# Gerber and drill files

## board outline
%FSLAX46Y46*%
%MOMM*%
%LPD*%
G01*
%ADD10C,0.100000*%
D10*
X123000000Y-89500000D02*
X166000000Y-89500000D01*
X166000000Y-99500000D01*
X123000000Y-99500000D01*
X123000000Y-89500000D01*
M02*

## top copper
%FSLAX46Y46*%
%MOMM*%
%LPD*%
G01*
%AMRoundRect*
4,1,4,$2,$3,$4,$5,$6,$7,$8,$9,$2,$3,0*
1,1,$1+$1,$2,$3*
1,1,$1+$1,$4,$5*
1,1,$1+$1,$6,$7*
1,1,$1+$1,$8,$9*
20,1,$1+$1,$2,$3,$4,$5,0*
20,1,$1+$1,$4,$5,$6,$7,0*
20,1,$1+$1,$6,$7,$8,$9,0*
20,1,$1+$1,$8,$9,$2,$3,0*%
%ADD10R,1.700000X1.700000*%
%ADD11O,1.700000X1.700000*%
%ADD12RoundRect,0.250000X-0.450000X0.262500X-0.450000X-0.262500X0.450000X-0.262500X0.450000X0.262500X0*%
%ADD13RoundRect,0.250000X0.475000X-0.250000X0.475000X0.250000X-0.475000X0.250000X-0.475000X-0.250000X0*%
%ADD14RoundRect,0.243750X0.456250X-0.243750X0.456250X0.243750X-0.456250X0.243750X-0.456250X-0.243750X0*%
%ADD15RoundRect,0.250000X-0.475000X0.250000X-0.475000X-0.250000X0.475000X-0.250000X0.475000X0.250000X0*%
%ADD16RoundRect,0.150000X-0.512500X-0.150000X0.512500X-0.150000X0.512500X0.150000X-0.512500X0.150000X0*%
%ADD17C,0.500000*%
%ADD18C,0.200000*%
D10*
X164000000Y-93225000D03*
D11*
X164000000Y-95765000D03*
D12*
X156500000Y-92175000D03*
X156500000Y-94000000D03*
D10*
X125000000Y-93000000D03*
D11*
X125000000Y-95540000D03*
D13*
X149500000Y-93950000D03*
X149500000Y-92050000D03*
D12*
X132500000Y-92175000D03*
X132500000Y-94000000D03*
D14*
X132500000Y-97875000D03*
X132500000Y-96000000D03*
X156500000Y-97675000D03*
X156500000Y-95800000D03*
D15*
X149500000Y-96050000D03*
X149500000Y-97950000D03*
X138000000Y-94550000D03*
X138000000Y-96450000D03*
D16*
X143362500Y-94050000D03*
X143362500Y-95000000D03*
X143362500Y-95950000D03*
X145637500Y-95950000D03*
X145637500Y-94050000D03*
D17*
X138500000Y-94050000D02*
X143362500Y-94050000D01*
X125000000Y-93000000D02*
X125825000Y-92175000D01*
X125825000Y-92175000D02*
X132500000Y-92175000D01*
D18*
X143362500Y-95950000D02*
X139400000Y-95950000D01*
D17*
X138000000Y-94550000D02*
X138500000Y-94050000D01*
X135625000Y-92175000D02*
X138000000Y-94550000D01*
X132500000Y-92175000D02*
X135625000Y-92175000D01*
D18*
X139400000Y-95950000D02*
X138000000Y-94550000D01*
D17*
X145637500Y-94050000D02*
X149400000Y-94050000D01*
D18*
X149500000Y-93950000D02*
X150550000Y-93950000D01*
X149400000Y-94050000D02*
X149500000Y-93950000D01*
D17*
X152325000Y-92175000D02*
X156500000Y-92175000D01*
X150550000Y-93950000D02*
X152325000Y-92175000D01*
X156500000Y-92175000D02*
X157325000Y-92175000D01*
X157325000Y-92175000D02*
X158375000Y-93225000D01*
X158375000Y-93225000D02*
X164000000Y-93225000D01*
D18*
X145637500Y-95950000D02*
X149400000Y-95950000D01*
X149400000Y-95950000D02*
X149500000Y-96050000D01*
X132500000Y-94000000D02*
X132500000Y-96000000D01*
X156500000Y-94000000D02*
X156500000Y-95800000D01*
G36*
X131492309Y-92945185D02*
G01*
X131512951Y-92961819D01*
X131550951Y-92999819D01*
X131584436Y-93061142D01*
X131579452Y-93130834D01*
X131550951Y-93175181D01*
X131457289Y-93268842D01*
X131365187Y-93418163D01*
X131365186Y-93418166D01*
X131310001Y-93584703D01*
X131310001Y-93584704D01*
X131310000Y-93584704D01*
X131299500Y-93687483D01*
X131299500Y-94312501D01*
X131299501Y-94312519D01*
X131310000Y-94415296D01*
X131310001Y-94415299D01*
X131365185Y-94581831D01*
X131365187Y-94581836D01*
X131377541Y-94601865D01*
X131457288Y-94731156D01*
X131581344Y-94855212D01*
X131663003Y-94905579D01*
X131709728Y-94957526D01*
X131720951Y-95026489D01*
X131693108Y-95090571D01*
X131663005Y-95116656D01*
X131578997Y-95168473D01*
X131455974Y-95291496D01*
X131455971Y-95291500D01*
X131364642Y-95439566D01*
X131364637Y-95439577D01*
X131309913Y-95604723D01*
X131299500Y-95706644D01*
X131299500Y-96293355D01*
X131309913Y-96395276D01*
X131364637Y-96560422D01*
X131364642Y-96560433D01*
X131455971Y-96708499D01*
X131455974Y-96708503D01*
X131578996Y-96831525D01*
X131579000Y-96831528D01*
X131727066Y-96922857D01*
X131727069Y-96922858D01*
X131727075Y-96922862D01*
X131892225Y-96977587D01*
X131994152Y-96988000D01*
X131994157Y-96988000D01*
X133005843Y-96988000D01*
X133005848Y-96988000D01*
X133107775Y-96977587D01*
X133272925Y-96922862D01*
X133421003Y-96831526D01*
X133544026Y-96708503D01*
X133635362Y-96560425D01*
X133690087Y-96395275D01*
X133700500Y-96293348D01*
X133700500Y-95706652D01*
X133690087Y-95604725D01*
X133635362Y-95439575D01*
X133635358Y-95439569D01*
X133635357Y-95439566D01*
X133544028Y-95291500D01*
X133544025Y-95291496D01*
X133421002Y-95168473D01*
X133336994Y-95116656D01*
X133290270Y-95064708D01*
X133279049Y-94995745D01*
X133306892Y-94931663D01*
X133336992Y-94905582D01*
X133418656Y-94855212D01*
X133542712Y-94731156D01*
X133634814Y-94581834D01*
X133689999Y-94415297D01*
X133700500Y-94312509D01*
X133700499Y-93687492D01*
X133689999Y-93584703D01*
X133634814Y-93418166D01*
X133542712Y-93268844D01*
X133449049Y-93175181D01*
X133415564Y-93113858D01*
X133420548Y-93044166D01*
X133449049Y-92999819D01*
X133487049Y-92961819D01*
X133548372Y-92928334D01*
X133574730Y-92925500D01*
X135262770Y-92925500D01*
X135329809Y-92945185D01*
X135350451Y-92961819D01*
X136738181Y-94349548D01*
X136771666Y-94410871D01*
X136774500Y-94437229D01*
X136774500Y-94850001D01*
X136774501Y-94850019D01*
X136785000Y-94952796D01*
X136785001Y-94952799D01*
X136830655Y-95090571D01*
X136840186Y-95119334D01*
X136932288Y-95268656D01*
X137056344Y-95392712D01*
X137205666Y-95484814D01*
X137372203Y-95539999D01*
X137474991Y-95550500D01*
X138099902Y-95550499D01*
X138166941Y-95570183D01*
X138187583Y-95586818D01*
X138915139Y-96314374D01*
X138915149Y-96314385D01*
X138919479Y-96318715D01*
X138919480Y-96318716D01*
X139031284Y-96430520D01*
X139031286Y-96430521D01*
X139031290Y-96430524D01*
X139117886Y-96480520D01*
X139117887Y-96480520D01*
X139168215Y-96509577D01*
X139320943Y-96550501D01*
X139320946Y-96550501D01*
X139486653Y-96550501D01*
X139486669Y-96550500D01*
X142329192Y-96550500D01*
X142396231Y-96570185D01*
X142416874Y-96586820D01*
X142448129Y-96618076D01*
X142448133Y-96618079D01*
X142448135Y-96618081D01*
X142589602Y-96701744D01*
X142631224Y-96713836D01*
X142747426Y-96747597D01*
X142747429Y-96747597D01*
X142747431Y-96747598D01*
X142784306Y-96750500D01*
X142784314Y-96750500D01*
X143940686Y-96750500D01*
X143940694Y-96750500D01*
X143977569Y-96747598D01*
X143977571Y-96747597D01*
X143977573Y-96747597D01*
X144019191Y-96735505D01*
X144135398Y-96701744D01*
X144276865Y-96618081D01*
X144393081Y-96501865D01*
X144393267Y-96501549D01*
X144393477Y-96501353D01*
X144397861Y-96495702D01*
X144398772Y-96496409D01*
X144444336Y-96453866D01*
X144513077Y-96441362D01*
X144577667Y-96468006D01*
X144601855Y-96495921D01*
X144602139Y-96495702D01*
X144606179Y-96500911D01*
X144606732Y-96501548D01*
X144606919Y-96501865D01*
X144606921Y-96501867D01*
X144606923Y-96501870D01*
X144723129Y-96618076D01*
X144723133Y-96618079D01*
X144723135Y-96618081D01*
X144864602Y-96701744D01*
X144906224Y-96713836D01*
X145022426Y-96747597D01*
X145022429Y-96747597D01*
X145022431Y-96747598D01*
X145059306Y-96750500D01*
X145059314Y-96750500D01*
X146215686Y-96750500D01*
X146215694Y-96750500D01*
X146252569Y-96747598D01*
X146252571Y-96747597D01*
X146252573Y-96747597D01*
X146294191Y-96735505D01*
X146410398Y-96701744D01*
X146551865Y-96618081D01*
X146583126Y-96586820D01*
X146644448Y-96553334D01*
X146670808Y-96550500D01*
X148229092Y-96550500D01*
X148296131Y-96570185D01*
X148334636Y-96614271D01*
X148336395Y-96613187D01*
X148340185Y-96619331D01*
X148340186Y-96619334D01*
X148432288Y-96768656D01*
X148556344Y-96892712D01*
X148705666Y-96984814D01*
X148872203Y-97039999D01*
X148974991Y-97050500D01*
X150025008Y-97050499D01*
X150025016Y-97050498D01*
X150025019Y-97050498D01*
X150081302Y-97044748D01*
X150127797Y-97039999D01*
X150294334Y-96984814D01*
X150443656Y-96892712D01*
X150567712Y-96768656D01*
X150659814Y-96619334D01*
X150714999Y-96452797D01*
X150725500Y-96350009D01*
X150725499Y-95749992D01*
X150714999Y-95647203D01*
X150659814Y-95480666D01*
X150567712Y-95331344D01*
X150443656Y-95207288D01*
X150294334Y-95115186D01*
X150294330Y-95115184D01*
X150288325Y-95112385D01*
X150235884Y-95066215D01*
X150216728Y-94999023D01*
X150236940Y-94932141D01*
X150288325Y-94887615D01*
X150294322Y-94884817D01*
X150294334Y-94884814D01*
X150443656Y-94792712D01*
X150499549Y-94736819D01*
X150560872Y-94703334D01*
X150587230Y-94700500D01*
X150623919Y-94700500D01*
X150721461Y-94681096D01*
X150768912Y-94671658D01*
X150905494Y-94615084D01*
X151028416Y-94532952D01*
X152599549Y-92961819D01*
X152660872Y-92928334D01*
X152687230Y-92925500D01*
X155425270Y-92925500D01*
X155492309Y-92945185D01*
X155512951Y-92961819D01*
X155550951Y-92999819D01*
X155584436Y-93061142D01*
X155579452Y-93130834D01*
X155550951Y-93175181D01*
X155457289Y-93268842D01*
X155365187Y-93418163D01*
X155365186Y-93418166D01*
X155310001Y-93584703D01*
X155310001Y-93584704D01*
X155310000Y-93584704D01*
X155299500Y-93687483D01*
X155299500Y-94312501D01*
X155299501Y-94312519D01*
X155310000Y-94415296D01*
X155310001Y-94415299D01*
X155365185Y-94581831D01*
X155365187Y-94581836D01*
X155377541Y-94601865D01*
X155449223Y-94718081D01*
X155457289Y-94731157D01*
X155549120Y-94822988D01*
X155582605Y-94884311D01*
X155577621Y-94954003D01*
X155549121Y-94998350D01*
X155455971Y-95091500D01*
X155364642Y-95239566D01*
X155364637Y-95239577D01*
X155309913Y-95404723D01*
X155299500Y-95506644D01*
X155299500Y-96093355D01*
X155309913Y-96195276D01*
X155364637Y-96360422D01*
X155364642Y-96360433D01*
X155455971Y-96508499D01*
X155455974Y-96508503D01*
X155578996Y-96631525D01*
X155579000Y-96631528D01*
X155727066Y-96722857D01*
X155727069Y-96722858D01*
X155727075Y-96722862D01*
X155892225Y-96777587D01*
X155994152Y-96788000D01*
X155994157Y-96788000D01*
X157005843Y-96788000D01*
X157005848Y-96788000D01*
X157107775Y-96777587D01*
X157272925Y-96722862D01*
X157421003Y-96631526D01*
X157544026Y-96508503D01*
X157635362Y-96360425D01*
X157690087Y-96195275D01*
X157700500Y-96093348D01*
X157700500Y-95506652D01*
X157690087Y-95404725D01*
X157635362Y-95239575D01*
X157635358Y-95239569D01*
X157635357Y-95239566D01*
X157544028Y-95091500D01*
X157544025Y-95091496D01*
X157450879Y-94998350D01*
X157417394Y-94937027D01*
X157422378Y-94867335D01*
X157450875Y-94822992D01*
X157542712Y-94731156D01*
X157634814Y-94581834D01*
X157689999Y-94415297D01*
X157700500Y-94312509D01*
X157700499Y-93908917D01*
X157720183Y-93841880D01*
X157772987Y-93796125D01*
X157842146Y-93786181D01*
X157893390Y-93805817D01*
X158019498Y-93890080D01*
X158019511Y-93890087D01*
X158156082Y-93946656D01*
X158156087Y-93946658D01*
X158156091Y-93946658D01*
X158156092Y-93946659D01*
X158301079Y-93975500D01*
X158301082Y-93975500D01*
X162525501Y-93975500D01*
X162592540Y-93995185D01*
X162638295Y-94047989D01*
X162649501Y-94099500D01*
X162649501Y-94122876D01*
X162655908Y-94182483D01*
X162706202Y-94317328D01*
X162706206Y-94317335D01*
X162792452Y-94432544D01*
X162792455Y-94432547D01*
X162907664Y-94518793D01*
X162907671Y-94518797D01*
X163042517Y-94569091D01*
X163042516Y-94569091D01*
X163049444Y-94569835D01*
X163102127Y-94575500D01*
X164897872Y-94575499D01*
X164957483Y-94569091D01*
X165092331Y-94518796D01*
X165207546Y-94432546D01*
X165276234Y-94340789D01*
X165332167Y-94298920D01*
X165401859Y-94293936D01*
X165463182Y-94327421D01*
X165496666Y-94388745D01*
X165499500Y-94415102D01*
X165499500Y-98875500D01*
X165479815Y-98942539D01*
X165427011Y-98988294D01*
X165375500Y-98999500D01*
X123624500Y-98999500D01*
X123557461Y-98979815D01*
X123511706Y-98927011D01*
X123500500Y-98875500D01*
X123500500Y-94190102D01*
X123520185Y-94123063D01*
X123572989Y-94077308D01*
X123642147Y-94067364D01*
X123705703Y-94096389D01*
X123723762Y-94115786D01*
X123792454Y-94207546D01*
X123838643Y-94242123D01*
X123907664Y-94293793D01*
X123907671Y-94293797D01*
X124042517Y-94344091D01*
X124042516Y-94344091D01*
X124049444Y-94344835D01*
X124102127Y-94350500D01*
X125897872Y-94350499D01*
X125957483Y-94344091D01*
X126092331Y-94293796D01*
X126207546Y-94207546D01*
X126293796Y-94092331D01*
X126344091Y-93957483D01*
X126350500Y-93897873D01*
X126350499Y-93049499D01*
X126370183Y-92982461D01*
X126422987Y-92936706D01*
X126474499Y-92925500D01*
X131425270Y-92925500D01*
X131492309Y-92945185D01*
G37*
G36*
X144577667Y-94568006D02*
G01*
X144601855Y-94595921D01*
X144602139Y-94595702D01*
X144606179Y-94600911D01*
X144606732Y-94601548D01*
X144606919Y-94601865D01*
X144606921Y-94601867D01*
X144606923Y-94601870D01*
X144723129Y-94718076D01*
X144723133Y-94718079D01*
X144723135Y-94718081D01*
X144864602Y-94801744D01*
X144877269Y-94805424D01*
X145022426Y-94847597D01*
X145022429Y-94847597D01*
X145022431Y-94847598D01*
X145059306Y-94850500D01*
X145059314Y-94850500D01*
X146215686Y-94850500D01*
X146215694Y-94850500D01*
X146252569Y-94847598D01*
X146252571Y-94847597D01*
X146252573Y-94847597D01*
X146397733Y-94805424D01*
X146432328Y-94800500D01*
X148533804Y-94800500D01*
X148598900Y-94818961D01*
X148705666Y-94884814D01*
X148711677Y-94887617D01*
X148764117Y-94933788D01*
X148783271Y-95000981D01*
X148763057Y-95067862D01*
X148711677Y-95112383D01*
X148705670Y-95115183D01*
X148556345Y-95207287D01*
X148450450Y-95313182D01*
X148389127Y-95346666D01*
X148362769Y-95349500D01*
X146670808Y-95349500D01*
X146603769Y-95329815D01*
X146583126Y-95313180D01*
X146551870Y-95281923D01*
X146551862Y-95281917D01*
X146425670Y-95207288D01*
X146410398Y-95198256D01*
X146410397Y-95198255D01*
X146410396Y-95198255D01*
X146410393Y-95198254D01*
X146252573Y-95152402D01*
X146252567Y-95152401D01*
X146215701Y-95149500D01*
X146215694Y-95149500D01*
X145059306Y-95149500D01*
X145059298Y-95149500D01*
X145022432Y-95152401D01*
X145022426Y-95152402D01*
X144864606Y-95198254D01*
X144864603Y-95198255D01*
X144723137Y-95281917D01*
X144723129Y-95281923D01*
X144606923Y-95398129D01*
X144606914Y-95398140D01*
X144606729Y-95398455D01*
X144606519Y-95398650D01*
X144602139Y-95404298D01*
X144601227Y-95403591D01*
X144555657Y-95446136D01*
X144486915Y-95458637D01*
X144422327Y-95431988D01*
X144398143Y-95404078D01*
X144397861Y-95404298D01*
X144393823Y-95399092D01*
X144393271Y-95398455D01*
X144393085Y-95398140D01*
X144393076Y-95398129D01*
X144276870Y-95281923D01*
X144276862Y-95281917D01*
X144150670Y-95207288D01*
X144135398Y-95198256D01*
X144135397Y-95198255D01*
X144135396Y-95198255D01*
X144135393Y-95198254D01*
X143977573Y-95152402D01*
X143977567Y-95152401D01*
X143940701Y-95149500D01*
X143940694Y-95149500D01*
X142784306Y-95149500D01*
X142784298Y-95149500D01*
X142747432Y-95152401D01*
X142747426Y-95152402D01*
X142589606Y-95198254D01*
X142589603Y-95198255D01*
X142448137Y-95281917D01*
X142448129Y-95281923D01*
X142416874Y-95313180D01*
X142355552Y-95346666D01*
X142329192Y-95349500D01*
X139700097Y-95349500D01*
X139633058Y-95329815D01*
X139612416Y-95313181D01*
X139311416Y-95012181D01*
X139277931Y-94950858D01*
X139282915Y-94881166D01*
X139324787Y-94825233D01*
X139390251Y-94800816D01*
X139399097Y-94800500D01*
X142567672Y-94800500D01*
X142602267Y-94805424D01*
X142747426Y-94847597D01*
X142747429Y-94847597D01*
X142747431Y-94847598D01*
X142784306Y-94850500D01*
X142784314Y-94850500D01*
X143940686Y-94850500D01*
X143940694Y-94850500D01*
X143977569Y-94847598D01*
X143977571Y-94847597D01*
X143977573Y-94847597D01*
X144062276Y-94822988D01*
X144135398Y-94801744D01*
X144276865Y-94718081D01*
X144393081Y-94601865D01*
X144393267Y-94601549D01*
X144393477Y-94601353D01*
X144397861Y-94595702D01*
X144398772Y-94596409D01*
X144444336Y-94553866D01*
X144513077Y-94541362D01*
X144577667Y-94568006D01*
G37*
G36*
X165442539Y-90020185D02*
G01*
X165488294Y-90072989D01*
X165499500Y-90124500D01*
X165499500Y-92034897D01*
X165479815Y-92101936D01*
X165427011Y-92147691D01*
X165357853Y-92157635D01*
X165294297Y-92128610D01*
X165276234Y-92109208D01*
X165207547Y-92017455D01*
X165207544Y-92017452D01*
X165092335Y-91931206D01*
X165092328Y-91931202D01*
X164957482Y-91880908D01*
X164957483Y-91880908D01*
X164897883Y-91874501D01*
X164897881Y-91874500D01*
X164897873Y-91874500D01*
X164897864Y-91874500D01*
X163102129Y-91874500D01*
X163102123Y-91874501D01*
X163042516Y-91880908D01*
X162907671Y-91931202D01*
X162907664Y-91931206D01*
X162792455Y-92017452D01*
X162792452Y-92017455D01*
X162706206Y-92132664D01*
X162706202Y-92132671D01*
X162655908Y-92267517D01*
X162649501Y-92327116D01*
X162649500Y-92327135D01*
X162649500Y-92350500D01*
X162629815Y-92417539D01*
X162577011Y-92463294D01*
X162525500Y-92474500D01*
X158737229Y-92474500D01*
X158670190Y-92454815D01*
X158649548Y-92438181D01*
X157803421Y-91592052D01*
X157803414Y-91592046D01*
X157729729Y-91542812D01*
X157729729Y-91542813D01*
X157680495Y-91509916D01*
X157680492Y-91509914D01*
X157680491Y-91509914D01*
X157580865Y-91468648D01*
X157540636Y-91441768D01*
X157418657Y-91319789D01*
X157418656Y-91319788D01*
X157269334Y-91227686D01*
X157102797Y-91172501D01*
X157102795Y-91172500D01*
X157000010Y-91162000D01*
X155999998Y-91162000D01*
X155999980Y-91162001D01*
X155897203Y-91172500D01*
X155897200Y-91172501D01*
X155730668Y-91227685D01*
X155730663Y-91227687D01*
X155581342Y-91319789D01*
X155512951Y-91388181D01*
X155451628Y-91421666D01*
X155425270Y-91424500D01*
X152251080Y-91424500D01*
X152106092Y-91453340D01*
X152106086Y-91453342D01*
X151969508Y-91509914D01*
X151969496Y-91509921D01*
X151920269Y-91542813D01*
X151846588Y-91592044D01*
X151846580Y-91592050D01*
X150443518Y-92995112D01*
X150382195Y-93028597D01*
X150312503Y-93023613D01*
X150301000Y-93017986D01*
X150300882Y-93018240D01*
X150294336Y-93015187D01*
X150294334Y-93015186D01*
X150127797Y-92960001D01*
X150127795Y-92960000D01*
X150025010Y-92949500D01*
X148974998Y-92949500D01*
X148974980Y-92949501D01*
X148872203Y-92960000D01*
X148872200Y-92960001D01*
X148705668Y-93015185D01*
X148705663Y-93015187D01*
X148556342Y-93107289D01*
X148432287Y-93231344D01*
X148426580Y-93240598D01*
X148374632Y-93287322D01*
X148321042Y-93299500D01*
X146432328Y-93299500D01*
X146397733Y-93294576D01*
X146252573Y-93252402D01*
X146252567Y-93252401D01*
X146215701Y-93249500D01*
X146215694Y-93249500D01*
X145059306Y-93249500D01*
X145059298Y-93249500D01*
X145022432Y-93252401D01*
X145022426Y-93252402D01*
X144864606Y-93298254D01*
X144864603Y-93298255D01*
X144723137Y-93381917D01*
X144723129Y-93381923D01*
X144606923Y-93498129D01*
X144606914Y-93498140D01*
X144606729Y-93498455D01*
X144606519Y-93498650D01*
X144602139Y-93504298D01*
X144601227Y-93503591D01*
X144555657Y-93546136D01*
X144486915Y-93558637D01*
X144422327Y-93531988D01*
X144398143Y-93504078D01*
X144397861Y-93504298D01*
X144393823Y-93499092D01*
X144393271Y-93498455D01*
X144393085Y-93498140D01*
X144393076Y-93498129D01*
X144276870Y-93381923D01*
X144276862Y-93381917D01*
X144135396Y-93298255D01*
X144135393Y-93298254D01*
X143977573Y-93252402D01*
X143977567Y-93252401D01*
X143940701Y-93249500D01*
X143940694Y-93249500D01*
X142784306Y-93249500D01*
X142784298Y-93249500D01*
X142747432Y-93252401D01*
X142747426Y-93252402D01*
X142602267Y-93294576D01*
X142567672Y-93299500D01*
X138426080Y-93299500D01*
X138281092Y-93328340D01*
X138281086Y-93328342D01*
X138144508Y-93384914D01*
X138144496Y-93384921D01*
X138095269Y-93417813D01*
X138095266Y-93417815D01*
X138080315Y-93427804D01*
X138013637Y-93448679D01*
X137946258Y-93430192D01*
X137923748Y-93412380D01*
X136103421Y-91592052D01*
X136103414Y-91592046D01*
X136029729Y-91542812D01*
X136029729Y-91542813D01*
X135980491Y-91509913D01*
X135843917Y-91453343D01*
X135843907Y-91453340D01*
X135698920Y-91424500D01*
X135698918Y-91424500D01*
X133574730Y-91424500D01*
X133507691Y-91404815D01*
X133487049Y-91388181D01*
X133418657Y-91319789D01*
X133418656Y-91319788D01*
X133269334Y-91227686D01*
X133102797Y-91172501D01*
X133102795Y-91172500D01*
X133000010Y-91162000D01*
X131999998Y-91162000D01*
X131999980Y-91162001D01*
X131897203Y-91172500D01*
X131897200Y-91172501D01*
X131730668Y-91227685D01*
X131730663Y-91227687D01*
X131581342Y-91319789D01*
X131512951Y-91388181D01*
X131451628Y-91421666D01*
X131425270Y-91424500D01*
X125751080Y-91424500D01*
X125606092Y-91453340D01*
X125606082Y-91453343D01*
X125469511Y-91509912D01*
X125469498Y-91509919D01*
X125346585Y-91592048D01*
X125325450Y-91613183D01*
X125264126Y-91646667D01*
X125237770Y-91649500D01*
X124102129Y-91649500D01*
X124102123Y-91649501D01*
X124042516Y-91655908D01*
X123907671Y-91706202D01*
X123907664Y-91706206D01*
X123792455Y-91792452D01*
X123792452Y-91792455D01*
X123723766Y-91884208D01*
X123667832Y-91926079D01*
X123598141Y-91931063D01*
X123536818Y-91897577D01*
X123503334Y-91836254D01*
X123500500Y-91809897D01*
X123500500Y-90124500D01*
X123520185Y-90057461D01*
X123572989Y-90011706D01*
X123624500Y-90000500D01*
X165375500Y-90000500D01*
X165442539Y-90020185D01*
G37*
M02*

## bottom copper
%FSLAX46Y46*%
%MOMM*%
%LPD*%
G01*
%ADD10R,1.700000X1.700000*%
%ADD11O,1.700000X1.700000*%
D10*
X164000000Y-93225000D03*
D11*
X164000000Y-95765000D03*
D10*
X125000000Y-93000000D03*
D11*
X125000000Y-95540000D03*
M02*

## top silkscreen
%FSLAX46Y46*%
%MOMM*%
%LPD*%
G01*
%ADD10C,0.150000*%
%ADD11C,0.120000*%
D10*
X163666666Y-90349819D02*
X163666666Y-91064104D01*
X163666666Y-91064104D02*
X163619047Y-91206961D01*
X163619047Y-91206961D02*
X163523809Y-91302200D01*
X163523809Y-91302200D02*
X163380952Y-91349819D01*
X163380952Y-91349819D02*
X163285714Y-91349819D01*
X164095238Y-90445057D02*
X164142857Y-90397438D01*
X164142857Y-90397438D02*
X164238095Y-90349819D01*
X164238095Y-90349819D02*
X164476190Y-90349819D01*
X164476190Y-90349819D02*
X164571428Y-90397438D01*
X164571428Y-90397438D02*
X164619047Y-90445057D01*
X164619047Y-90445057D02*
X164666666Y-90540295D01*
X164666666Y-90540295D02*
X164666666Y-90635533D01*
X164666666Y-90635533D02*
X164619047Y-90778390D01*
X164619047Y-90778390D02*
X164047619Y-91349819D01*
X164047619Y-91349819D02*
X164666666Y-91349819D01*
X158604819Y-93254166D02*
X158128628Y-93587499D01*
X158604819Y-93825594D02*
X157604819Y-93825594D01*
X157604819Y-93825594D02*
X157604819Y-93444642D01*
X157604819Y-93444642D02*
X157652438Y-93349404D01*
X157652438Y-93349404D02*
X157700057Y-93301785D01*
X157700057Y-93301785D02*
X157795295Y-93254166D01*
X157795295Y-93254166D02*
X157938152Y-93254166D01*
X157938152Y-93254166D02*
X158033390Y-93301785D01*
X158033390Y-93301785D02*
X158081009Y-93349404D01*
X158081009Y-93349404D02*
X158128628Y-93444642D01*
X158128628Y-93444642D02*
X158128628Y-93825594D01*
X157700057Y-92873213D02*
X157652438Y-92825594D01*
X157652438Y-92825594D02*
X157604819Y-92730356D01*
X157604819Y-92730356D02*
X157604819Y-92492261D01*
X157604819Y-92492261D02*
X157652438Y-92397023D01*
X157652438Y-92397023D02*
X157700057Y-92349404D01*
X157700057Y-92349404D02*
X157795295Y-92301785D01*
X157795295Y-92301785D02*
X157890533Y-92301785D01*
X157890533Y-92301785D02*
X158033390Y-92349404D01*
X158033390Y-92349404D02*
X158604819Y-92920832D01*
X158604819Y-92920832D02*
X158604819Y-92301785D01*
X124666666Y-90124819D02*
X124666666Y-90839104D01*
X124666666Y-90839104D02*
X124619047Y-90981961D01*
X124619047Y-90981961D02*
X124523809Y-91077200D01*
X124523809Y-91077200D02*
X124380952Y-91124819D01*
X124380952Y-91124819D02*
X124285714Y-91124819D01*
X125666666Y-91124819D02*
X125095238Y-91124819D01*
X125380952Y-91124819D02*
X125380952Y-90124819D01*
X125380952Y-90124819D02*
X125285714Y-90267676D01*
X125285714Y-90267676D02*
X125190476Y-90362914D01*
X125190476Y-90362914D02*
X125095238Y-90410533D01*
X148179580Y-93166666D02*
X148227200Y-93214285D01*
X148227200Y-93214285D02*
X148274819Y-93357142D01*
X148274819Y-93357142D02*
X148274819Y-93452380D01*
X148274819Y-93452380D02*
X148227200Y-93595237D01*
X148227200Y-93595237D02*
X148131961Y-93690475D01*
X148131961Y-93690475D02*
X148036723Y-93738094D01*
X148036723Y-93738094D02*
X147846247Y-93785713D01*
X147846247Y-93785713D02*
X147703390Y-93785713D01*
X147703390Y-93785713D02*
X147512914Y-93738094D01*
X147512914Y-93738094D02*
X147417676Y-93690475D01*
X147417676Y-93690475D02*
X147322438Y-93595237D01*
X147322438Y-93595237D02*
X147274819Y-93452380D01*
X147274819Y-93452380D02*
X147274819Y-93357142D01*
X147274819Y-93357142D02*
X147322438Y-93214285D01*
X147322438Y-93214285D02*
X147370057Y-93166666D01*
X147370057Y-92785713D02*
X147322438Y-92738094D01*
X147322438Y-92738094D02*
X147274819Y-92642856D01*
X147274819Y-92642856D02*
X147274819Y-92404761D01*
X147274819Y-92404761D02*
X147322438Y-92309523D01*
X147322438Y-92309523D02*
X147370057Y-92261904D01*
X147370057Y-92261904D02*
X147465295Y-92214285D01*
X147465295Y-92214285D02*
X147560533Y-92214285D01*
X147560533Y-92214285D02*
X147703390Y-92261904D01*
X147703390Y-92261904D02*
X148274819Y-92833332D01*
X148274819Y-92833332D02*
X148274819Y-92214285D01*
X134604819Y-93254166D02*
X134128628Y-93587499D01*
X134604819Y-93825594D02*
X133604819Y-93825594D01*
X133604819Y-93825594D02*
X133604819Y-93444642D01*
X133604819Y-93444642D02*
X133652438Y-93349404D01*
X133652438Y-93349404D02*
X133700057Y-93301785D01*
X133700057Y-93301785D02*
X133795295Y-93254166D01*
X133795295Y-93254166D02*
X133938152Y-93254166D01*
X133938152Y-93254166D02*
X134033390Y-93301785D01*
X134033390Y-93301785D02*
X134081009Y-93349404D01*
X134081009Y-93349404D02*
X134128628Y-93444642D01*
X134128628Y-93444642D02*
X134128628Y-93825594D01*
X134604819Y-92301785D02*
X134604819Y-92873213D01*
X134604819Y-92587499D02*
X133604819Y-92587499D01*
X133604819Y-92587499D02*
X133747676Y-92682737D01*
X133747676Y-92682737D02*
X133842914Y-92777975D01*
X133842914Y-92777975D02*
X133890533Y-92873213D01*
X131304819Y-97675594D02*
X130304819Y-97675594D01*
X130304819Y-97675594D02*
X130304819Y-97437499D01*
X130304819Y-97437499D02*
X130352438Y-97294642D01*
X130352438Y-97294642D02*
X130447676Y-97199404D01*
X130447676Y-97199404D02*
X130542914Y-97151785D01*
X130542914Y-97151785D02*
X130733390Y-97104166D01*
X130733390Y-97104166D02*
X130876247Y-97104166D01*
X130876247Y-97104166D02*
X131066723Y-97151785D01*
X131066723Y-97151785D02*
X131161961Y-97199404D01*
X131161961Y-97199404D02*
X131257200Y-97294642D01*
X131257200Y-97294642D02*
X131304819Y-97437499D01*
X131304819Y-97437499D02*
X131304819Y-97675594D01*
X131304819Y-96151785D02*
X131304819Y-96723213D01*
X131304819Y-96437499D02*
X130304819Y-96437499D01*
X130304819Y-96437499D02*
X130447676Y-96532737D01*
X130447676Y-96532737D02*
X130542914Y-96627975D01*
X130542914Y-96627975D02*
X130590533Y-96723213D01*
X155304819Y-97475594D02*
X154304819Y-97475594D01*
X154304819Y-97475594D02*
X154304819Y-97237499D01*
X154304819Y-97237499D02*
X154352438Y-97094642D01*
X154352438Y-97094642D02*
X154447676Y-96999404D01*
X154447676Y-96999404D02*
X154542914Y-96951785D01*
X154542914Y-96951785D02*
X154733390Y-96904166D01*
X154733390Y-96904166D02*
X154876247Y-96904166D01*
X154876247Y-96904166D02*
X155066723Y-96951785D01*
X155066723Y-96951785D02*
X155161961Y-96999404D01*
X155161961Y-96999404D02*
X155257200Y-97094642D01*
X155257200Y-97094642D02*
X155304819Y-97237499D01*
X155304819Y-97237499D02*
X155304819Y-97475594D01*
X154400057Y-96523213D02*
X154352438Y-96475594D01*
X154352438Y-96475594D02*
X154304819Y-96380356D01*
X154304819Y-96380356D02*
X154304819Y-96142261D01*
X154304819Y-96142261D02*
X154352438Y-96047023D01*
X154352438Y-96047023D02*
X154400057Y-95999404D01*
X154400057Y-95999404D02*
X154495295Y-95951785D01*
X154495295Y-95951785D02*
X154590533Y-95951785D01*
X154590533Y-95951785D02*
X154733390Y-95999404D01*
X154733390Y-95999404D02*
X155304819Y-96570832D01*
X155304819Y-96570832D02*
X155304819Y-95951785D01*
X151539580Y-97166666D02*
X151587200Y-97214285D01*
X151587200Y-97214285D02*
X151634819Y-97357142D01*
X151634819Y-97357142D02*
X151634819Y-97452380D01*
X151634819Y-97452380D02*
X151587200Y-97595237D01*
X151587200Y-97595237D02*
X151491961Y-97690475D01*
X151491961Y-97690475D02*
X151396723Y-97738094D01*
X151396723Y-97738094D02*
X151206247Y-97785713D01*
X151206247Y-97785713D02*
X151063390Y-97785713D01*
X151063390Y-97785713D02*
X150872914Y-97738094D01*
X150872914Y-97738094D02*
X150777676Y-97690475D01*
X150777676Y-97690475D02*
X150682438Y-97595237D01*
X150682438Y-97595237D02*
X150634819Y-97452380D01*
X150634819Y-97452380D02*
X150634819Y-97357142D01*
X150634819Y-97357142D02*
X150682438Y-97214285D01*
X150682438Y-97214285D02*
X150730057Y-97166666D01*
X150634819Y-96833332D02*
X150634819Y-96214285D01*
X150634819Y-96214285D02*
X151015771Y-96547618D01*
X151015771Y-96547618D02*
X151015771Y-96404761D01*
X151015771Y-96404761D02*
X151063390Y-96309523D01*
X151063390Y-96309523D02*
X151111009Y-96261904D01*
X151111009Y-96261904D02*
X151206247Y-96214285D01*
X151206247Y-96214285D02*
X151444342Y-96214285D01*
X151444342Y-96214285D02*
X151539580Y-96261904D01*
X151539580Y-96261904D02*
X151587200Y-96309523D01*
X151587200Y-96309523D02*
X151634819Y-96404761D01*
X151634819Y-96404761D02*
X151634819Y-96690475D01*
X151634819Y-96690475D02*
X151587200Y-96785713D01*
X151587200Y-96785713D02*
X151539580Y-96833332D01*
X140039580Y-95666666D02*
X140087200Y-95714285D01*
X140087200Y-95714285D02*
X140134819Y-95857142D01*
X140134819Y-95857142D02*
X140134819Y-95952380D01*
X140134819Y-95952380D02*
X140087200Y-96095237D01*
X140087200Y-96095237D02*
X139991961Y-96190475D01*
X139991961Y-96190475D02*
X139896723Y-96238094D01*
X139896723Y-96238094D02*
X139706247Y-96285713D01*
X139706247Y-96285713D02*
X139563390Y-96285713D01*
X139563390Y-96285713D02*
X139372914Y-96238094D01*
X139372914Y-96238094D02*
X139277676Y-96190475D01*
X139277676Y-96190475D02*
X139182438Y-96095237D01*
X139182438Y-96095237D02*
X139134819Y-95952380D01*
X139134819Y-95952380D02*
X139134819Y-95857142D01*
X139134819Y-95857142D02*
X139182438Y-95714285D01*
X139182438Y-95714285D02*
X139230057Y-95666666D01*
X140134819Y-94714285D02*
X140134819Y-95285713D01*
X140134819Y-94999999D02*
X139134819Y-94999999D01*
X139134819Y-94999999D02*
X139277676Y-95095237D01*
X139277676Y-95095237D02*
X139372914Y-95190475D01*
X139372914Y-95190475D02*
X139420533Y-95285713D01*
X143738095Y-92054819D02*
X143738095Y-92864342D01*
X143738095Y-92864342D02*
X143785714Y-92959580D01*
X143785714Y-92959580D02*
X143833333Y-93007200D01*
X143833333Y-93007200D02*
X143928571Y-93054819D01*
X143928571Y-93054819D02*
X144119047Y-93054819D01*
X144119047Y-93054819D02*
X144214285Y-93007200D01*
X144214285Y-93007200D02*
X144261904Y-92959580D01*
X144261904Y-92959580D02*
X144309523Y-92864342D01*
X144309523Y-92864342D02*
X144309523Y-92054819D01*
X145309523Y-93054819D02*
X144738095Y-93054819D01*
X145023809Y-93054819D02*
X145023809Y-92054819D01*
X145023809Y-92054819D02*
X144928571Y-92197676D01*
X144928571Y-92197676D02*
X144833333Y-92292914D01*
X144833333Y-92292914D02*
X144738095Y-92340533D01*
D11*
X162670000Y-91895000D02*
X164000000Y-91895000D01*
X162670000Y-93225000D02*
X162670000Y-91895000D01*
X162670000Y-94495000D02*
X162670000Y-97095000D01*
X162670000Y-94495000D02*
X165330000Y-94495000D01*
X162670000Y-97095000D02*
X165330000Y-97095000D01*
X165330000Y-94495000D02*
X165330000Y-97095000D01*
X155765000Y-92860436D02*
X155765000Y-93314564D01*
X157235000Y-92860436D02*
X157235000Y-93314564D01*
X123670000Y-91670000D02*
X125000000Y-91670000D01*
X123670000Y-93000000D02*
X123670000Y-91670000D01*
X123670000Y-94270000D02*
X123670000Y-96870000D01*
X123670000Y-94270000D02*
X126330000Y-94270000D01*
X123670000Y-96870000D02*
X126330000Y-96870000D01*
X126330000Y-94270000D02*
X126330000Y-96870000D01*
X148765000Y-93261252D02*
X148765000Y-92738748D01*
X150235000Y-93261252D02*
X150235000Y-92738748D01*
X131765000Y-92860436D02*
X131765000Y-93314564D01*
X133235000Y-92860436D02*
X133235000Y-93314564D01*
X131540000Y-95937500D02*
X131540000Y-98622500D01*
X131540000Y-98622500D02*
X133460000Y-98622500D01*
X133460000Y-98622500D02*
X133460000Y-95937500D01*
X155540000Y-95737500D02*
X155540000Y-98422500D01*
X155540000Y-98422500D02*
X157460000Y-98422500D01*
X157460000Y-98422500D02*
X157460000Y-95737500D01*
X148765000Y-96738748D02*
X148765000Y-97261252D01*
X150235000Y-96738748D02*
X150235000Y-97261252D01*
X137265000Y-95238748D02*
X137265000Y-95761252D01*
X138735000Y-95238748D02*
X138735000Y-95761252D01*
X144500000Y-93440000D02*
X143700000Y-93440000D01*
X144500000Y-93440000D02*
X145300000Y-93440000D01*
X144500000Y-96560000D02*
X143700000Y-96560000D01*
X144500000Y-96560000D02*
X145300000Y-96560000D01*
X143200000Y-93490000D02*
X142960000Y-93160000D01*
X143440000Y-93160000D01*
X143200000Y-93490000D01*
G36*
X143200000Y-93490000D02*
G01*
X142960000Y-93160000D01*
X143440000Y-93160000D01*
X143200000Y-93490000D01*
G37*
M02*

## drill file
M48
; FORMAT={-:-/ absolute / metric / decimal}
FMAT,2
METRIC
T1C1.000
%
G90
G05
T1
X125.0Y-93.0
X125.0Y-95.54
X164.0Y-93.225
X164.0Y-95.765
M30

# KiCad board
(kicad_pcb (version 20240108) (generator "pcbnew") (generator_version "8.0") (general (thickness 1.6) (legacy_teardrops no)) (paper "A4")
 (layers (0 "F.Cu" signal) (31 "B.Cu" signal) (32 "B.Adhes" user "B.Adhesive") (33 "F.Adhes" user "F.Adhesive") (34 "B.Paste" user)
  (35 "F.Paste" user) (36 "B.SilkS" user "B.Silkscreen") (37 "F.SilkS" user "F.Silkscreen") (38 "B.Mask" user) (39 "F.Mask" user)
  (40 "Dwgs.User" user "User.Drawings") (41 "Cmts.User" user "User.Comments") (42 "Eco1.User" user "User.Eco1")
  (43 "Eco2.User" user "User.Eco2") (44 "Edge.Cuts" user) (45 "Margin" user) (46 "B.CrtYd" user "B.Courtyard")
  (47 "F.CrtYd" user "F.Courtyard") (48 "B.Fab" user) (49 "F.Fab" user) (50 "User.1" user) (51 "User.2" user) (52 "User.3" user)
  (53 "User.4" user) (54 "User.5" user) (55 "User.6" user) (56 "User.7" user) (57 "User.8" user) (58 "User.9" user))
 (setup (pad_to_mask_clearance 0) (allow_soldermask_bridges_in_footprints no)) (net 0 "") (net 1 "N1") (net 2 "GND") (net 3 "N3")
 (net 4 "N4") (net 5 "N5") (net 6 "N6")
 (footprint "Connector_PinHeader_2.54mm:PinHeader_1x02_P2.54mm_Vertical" (layer "F.Cu") (at 164 93.225)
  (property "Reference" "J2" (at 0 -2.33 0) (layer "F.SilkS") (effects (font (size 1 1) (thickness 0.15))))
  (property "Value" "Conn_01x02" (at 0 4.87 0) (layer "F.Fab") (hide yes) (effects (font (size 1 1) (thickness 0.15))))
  (fp_line (start -1.33 -1.33) (end 0 -1.33) (stroke (width 0.12) (type solid)) (layer "F.SilkS"))
  (fp_line (start -1.33 0) (end -1.33 -1.33) (stroke (width 0.12) (type solid)) (layer "F.SilkS"))
  (fp_line (start -1.33 1.27) (end -1.33 3.87) (stroke (width 0.12) (type solid)) (layer "F.SilkS"))
  (fp_line (start -1.33 1.27) (end 1.33 1.27) (stroke (width 0.12) (type solid)) (layer "F.SilkS"))
  (fp_line (start -1.33 3.87) (end 1.33 3.87) (stroke (width 0.12) (type solid)) (layer "F.SilkS"))
  (fp_line (start 1.33 1.27) (end 1.33 3.87) (stroke (width 0.12) (type solid)) (layer "F.SilkS"))
  (pad "1" thru_hole rect (at 0 0) (size 1.7 1.7) (drill 1) (layers "*.Cu" "*.Mask") (remove_unused_layers no) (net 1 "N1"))
  (pad "2" thru_hole oval (at 0 2.54) (size 1.7 1.7) (drill 1) (layers "*.Cu" "*.Mask") (remove_unused_layers no) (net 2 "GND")))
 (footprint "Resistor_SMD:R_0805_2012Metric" (layer "F.Cu") (at 156.5 93.0875 -90)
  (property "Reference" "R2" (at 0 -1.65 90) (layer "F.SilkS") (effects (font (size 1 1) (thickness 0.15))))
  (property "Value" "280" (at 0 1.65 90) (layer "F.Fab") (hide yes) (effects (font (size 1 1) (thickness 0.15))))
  (fp_line (start -0.227064 0.735) (end 0.227064 0.735) (stroke (width 0.12) (type solid)) (layer "F.SilkS"))
  (fp_line (start -0.227064 -0.735) (end 0.227064 -0.735) (stroke (width 0.12) (type solid)) (layer "F.SilkS"))
  (pad "1" smd roundrect (at -0.9125 0 270) (size 1.025 1.4) (layers "F.Cu" "F.Paste" "F.Mask") (roundrect_rratio 0.243902) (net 1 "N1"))
  (pad "2" smd roundrect (at 0.9125 0 270) (size 1.025 1.4) (layers "F.Cu" "F.Paste" "F.Mask") (roundrect_rratio 0.243902) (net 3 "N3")))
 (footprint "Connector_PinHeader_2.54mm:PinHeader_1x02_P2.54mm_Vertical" (layer "F.Cu") (at 125 93)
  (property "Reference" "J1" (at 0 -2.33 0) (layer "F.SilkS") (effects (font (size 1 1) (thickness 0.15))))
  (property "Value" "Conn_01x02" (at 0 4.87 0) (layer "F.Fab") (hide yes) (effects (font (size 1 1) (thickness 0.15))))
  (fp_line (start -1.33 -1.33) (end 0 -1.33) (stroke (width 0.12) (type solid)) (layer "F.SilkS"))
  (fp_line (start -1.33 0) (end -1.33 -1.33) (stroke (width 0.12) (type solid)) (layer "F.SilkS"))
  (fp_line (start -1.33 1.27) (end -1.33 3.87) (stroke (width 0.12) (type solid)) (layer "F.SilkS"))
  (fp_line (start -1.33 1.27) (end 1.33 1.27) (stroke (width 0.12) (type solid)) (layer "F.SilkS"))
  (fp_line (start -1.33 3.87) (end 1.33 3.87) (stroke (width 0.12) (type solid)) (layer "F.SilkS"))
  (fp_line (start 1.33 1.27) (end 1.33 3.87) (stroke (width 0.12) (type solid)) (layer "F.SilkS"))
  (pad "1" thru_hole rect (at 0 0) (size 1.7 1.7) (drill 1) (layers "*.Cu" "*.Mask") (remove_unused_layers no) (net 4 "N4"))
  (pad "2" thru_hole oval (at 0 2.54) (size 1.7 1.7) (drill 1) (layers "*.Cu" "*.Mask") (remove_unused_layers no) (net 2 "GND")))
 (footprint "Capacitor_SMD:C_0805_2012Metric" (layer "F.Cu") (at 149.5 93 90)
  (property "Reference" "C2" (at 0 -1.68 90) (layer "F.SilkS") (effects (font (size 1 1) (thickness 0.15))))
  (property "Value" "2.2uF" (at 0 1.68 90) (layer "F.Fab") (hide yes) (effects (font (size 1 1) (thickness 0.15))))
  (fp_line (start -0.261252 -0.735) (end 0.261252 -0.735) (stroke (width 0.12) (type solid)) (layer "F.SilkS"))
  (fp_line (start -0.261252 0.735) (end 0.261252 0.735) (stroke (width 0.12) (type solid)) (layer "F.SilkS"))
  (pad "1" smd roundrect (at -0.95 0 90) (size 1 1.45) (layers "F.Cu" "F.Paste" "F.Mask") (roundrect_rratio 0.25) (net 1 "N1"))
  (pad "2" smd roundrect (at 0.95 0 90) (size 1 1.45) (layers "F.Cu" "F.Paste" "F.Mask") (roundrect_rratio 0.25) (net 2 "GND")))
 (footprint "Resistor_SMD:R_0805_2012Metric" (layer "F.Cu") (at 132.5 93.0875 -90)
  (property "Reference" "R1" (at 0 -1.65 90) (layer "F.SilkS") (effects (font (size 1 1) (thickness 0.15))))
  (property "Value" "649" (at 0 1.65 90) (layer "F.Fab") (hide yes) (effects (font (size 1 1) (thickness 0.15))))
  (fp_line (start -0.227064 0.735) (end 0.227064 0.735) (stroke (width 0.12) (type solid)) (layer "F.SilkS"))
  (fp_line (start -0.227064 -0.735) (end 0.227064 -0.735) (stroke (width 0.12) (type solid)) (layer "F.SilkS"))
  (pad "1" smd roundrect (at -0.9125 0 270) (size 1.025 1.4) (layers "F.Cu" "F.Paste" "F.Mask") (roundrect_rratio 0.243902) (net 4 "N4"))
  (pad "2" smd roundrect (at 0.9125 0 270) (size 1.025 1.4) (layers "F.Cu" "F.Paste" "F.Mask") (roundrect_rratio 0.243902) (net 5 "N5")))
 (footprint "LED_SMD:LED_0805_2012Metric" (layer "F.Cu") (at 132.5 96.9375 90)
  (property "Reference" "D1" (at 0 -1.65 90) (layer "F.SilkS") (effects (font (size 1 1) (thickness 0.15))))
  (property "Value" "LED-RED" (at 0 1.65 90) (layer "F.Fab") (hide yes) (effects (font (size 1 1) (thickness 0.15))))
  (fp_line (start 1 -0.96) (end -1.685 -0.96) (stroke (width 0.12) (type solid)) (layer "F.SilkS"))
  (fp_line (start -1.685 -0.96) (end -1.685 0.96) (stroke (width 0.12) (type solid)) (layer "F.SilkS"))
  (fp_line (start -1.685 0.96) (end 1 0.96) (stroke (width 0.12) (type solid)) (layer "F.SilkS"))
  (pad "1" smd roundrect (at -0.9375 0 90) (size 0.975 1.4) (layers "F.Cu" "F.Paste" "F.Mask") (roundrect_rratio 0.25) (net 2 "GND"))
  (pad "2" smd roundrect (at 0.9375 0 90) (size 0.975 1.4) (layers "F.Cu" "F.Paste" "F.Mask") (roundrect_rratio 0.25) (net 5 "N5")))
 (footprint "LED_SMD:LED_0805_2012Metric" (layer "F.Cu") (at 156.5 96.7375 90)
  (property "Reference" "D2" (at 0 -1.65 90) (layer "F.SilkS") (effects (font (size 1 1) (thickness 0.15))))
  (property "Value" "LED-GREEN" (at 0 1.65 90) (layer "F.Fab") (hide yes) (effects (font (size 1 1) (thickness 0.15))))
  (fp_line (start 1 -0.96) (end -1.685 -0.96) (stroke (width 0.12) (type solid)) (layer "F.SilkS"))
  (fp_line (start -1.685 -0.96) (end -1.685 0.96) (stroke (width 0.12) (type solid)) (layer "F.SilkS"))
  (fp_line (start -1.685 0.96) (end 1 0.96) (stroke (width 0.12) (type solid)) (layer "F.SilkS"))
  (pad "1" smd roundrect (at -0.9375 0 90) (size 0.975 1.4) (layers "F.Cu" "F.Paste" "F.Mask") (roundrect_rratio 0.25) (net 2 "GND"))
  (pad "2" smd roundrect (at 0.9375 0 90) (size 0.975 1.4) (layers "F.Cu" "F.Paste" "F.Mask") (roundrect_rratio 0.25) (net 3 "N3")))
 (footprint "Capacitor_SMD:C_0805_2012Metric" (layer "F.Cu") (at 149.5 97 -90)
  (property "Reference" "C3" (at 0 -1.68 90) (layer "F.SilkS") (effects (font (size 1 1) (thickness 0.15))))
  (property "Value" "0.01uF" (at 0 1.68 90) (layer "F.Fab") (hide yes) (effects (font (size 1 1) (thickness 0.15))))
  (fp_line (start -0.261252 0.735) (end 0.261252 0.735) (stroke (width 0.12) (type solid)) (layer "F.SilkS"))
  (fp_line (start -0.261252 -0.735) (end 0.261252 -0.735) (stroke (width 0.12) (type solid)) (layer "F.SilkS"))
  (pad "1" smd roundrect (at -0.95 0 270) (size 1 1.45) (layers "F.Cu" "F.Paste" "F.Mask") (roundrect_rratio 0.25) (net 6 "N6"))
  (pad "2" smd roundrect (at 0.95 0 270) (size 1 1.45) (layers "F.Cu" "F.Paste" "F.Mask") (roundrect_rratio 0.25) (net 2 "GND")))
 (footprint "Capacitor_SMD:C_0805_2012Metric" (layer "F.Cu") (at 138 95.5 -90)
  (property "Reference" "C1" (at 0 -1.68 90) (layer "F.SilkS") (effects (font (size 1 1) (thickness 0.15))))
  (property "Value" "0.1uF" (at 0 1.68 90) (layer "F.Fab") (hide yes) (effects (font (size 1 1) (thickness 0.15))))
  (fp_line (start -0.261252 0.735) (end 0.261252 0.735) (stroke (width 0.12) (type solid)) (layer "F.SilkS"))
  (fp_line (start -0.261252 -0.735) (end 0.261252 -0.735) (stroke (width 0.12) (type solid)) (layer "F.SilkS"))
  (pad "1" smd roundrect (at -0.95 0 270) (size 1 1.45) (layers "F.Cu" "F.Paste" "F.Mask") (roundrect_rratio 0.25) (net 4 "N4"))
  (pad "2" smd roundrect (at 0.95 0 270) (size 1 1.45) (layers "F.Cu" "F.Paste" "F.Mask") (roundrect_rratio 0.25) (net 2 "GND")))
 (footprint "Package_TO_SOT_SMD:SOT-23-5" (layer "F.Cu") (at 144.5 95)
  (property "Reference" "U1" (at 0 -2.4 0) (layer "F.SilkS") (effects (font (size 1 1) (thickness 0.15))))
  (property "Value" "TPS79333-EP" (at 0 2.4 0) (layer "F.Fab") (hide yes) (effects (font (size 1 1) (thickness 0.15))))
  (fp_line (start 0 -1.56) (end -0.8 -1.56) (stroke (width 0.12) (type solid)) (layer "F.SilkS"))
  (fp_line (start 0 -1.56) (end 0.8 -1.56) (stroke (width 0.12) (type solid)) (layer "F.SilkS"))
  (fp_line (start 0 1.56) (end -0.8 1.56) (stroke (width 0.12) (type solid)) (layer "F.SilkS"))
  (fp_line (start 0 1.56) (end 0.8 1.56) (stroke (width 0.12) (type solid)) (layer "F.SilkS"))
  (fp_poly
   (pts (xy -1.3 -1.51) (xy -1.54 -1.84) (xy -1.06 -1.84) (xy -1.3 -1.51)) (stroke (width 0.12) (type solid)) (fill solid) (layer "F.SilkS"))
  (pad "1" smd roundrect (at -1.1375 -0.95) (size 1.325 0.6) (layers "F.Cu" "F.Paste" "F.Mask") (roundrect_rratio 0.25) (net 4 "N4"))
  (pad "2" smd roundrect (at -1.1375 0) (size 1.325 0.6) (layers "F.Cu" "F.Paste" "F.Mask") (roundrect_rratio 0.25) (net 2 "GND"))
  (pad "3" smd roundrect (at -1.1375 0.95) (size 1.325 0.6) (layers "F.Cu" "F.Paste" "F.Mask") (roundrect_rratio 0.25) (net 4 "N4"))
  (pad "4" smd roundrect (at 1.1375 0.95) (size 1.325 0.6) (layers "F.Cu" "F.Paste" "F.Mask") (roundrect_rratio 0.25) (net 6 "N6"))
  (pad "5" smd roundrect (at 1.1375 -0.95) (size 1.325 0.6) (layers "F.Cu" "F.Paste" "F.Mask") (roundrect_rratio 0.25) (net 1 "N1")))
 (gr_rect (start 123 89.5) (end 166 99.5) (stroke (width 0.1) (type default)) (fill none) (layer "Edge.Cuts"))
 (segment (start 138.5 94.05) (end 143.3625 94.05) (width 0.5) (layer "F.Cu") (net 4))
 (segment (start 125 93) (end 125.825 92.175) (width 0.5) (layer "F.Cu") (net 4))
 (segment (start 125.825 92.175) (end 132.5 92.175) (width 0.5) (layer "F.Cu") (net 4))
 (segment (start 143.3625 95.95) (end 139.4 95.95) (width 0.2) (layer "F.Cu") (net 4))
 (segment (start 138 94.55) (end 138.5 94.05) (width 0.5) (layer "F.Cu") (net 4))
 (segment (start 135.625 92.175) (end 138 94.55) (width 0.5) (layer "F.Cu") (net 4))
 (segment (start 132.5 92.175) (end 135.625 92.175) (width 0.5) (layer "F.Cu") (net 4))
 (segment (start 139.4 95.95) (end 138 94.55) (width 0.2) (layer "F.Cu") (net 4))
 (segment (start 145.6375 94.05) (end 149.4 94.05) (width 0.5) (layer "F.Cu") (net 1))
 (segment (start 149.5 93.95) (end 150.55 93.95) (width 0.2) (layer "F.Cu") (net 1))
 (segment (start 149.4 94.05) (end 149.5 93.95) (width 0.2) (layer "F.Cu") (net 1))
 (segment (start 152.325 92.175) (end 156.5 92.175) (width 0.5) (layer "F.Cu") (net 1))
 (segment (start 150.55 93.95) (end 152.325 92.175) (width 0.5) (layer "F.Cu") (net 1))
 (segment (start 156.5 92.175) (end 157.325 92.175) (width 0.5) (layer "F.Cu") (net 1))
 (segment (start 157.325 92.175) (end 158.375 93.225) (width 0.5) (layer "F.Cu") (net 1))
 (segment (start 158.375 93.225) (end 164 93.225) (width 0.5) (layer "F.Cu") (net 1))
 (segment (start 145.6375 95.95) (end 149.4 95.95) (width 0.2) (layer "F.Cu") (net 6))
 (segment (start 149.4 95.95) (end 149.5 96.05) (width 0.2) (layer "F.Cu") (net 6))
 (segment (start 132.5 94) (end 132.5 96) (width 0.2) (layer "F.Cu") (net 5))
 (segment (start 156.5 94) (end 156.5 95.8) (width 0.2) (layer "F.Cu") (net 3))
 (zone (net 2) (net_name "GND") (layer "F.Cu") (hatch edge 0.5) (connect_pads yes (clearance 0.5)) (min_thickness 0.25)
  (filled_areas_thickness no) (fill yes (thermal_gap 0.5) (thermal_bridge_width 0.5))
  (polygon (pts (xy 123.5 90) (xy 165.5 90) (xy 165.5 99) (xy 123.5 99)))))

